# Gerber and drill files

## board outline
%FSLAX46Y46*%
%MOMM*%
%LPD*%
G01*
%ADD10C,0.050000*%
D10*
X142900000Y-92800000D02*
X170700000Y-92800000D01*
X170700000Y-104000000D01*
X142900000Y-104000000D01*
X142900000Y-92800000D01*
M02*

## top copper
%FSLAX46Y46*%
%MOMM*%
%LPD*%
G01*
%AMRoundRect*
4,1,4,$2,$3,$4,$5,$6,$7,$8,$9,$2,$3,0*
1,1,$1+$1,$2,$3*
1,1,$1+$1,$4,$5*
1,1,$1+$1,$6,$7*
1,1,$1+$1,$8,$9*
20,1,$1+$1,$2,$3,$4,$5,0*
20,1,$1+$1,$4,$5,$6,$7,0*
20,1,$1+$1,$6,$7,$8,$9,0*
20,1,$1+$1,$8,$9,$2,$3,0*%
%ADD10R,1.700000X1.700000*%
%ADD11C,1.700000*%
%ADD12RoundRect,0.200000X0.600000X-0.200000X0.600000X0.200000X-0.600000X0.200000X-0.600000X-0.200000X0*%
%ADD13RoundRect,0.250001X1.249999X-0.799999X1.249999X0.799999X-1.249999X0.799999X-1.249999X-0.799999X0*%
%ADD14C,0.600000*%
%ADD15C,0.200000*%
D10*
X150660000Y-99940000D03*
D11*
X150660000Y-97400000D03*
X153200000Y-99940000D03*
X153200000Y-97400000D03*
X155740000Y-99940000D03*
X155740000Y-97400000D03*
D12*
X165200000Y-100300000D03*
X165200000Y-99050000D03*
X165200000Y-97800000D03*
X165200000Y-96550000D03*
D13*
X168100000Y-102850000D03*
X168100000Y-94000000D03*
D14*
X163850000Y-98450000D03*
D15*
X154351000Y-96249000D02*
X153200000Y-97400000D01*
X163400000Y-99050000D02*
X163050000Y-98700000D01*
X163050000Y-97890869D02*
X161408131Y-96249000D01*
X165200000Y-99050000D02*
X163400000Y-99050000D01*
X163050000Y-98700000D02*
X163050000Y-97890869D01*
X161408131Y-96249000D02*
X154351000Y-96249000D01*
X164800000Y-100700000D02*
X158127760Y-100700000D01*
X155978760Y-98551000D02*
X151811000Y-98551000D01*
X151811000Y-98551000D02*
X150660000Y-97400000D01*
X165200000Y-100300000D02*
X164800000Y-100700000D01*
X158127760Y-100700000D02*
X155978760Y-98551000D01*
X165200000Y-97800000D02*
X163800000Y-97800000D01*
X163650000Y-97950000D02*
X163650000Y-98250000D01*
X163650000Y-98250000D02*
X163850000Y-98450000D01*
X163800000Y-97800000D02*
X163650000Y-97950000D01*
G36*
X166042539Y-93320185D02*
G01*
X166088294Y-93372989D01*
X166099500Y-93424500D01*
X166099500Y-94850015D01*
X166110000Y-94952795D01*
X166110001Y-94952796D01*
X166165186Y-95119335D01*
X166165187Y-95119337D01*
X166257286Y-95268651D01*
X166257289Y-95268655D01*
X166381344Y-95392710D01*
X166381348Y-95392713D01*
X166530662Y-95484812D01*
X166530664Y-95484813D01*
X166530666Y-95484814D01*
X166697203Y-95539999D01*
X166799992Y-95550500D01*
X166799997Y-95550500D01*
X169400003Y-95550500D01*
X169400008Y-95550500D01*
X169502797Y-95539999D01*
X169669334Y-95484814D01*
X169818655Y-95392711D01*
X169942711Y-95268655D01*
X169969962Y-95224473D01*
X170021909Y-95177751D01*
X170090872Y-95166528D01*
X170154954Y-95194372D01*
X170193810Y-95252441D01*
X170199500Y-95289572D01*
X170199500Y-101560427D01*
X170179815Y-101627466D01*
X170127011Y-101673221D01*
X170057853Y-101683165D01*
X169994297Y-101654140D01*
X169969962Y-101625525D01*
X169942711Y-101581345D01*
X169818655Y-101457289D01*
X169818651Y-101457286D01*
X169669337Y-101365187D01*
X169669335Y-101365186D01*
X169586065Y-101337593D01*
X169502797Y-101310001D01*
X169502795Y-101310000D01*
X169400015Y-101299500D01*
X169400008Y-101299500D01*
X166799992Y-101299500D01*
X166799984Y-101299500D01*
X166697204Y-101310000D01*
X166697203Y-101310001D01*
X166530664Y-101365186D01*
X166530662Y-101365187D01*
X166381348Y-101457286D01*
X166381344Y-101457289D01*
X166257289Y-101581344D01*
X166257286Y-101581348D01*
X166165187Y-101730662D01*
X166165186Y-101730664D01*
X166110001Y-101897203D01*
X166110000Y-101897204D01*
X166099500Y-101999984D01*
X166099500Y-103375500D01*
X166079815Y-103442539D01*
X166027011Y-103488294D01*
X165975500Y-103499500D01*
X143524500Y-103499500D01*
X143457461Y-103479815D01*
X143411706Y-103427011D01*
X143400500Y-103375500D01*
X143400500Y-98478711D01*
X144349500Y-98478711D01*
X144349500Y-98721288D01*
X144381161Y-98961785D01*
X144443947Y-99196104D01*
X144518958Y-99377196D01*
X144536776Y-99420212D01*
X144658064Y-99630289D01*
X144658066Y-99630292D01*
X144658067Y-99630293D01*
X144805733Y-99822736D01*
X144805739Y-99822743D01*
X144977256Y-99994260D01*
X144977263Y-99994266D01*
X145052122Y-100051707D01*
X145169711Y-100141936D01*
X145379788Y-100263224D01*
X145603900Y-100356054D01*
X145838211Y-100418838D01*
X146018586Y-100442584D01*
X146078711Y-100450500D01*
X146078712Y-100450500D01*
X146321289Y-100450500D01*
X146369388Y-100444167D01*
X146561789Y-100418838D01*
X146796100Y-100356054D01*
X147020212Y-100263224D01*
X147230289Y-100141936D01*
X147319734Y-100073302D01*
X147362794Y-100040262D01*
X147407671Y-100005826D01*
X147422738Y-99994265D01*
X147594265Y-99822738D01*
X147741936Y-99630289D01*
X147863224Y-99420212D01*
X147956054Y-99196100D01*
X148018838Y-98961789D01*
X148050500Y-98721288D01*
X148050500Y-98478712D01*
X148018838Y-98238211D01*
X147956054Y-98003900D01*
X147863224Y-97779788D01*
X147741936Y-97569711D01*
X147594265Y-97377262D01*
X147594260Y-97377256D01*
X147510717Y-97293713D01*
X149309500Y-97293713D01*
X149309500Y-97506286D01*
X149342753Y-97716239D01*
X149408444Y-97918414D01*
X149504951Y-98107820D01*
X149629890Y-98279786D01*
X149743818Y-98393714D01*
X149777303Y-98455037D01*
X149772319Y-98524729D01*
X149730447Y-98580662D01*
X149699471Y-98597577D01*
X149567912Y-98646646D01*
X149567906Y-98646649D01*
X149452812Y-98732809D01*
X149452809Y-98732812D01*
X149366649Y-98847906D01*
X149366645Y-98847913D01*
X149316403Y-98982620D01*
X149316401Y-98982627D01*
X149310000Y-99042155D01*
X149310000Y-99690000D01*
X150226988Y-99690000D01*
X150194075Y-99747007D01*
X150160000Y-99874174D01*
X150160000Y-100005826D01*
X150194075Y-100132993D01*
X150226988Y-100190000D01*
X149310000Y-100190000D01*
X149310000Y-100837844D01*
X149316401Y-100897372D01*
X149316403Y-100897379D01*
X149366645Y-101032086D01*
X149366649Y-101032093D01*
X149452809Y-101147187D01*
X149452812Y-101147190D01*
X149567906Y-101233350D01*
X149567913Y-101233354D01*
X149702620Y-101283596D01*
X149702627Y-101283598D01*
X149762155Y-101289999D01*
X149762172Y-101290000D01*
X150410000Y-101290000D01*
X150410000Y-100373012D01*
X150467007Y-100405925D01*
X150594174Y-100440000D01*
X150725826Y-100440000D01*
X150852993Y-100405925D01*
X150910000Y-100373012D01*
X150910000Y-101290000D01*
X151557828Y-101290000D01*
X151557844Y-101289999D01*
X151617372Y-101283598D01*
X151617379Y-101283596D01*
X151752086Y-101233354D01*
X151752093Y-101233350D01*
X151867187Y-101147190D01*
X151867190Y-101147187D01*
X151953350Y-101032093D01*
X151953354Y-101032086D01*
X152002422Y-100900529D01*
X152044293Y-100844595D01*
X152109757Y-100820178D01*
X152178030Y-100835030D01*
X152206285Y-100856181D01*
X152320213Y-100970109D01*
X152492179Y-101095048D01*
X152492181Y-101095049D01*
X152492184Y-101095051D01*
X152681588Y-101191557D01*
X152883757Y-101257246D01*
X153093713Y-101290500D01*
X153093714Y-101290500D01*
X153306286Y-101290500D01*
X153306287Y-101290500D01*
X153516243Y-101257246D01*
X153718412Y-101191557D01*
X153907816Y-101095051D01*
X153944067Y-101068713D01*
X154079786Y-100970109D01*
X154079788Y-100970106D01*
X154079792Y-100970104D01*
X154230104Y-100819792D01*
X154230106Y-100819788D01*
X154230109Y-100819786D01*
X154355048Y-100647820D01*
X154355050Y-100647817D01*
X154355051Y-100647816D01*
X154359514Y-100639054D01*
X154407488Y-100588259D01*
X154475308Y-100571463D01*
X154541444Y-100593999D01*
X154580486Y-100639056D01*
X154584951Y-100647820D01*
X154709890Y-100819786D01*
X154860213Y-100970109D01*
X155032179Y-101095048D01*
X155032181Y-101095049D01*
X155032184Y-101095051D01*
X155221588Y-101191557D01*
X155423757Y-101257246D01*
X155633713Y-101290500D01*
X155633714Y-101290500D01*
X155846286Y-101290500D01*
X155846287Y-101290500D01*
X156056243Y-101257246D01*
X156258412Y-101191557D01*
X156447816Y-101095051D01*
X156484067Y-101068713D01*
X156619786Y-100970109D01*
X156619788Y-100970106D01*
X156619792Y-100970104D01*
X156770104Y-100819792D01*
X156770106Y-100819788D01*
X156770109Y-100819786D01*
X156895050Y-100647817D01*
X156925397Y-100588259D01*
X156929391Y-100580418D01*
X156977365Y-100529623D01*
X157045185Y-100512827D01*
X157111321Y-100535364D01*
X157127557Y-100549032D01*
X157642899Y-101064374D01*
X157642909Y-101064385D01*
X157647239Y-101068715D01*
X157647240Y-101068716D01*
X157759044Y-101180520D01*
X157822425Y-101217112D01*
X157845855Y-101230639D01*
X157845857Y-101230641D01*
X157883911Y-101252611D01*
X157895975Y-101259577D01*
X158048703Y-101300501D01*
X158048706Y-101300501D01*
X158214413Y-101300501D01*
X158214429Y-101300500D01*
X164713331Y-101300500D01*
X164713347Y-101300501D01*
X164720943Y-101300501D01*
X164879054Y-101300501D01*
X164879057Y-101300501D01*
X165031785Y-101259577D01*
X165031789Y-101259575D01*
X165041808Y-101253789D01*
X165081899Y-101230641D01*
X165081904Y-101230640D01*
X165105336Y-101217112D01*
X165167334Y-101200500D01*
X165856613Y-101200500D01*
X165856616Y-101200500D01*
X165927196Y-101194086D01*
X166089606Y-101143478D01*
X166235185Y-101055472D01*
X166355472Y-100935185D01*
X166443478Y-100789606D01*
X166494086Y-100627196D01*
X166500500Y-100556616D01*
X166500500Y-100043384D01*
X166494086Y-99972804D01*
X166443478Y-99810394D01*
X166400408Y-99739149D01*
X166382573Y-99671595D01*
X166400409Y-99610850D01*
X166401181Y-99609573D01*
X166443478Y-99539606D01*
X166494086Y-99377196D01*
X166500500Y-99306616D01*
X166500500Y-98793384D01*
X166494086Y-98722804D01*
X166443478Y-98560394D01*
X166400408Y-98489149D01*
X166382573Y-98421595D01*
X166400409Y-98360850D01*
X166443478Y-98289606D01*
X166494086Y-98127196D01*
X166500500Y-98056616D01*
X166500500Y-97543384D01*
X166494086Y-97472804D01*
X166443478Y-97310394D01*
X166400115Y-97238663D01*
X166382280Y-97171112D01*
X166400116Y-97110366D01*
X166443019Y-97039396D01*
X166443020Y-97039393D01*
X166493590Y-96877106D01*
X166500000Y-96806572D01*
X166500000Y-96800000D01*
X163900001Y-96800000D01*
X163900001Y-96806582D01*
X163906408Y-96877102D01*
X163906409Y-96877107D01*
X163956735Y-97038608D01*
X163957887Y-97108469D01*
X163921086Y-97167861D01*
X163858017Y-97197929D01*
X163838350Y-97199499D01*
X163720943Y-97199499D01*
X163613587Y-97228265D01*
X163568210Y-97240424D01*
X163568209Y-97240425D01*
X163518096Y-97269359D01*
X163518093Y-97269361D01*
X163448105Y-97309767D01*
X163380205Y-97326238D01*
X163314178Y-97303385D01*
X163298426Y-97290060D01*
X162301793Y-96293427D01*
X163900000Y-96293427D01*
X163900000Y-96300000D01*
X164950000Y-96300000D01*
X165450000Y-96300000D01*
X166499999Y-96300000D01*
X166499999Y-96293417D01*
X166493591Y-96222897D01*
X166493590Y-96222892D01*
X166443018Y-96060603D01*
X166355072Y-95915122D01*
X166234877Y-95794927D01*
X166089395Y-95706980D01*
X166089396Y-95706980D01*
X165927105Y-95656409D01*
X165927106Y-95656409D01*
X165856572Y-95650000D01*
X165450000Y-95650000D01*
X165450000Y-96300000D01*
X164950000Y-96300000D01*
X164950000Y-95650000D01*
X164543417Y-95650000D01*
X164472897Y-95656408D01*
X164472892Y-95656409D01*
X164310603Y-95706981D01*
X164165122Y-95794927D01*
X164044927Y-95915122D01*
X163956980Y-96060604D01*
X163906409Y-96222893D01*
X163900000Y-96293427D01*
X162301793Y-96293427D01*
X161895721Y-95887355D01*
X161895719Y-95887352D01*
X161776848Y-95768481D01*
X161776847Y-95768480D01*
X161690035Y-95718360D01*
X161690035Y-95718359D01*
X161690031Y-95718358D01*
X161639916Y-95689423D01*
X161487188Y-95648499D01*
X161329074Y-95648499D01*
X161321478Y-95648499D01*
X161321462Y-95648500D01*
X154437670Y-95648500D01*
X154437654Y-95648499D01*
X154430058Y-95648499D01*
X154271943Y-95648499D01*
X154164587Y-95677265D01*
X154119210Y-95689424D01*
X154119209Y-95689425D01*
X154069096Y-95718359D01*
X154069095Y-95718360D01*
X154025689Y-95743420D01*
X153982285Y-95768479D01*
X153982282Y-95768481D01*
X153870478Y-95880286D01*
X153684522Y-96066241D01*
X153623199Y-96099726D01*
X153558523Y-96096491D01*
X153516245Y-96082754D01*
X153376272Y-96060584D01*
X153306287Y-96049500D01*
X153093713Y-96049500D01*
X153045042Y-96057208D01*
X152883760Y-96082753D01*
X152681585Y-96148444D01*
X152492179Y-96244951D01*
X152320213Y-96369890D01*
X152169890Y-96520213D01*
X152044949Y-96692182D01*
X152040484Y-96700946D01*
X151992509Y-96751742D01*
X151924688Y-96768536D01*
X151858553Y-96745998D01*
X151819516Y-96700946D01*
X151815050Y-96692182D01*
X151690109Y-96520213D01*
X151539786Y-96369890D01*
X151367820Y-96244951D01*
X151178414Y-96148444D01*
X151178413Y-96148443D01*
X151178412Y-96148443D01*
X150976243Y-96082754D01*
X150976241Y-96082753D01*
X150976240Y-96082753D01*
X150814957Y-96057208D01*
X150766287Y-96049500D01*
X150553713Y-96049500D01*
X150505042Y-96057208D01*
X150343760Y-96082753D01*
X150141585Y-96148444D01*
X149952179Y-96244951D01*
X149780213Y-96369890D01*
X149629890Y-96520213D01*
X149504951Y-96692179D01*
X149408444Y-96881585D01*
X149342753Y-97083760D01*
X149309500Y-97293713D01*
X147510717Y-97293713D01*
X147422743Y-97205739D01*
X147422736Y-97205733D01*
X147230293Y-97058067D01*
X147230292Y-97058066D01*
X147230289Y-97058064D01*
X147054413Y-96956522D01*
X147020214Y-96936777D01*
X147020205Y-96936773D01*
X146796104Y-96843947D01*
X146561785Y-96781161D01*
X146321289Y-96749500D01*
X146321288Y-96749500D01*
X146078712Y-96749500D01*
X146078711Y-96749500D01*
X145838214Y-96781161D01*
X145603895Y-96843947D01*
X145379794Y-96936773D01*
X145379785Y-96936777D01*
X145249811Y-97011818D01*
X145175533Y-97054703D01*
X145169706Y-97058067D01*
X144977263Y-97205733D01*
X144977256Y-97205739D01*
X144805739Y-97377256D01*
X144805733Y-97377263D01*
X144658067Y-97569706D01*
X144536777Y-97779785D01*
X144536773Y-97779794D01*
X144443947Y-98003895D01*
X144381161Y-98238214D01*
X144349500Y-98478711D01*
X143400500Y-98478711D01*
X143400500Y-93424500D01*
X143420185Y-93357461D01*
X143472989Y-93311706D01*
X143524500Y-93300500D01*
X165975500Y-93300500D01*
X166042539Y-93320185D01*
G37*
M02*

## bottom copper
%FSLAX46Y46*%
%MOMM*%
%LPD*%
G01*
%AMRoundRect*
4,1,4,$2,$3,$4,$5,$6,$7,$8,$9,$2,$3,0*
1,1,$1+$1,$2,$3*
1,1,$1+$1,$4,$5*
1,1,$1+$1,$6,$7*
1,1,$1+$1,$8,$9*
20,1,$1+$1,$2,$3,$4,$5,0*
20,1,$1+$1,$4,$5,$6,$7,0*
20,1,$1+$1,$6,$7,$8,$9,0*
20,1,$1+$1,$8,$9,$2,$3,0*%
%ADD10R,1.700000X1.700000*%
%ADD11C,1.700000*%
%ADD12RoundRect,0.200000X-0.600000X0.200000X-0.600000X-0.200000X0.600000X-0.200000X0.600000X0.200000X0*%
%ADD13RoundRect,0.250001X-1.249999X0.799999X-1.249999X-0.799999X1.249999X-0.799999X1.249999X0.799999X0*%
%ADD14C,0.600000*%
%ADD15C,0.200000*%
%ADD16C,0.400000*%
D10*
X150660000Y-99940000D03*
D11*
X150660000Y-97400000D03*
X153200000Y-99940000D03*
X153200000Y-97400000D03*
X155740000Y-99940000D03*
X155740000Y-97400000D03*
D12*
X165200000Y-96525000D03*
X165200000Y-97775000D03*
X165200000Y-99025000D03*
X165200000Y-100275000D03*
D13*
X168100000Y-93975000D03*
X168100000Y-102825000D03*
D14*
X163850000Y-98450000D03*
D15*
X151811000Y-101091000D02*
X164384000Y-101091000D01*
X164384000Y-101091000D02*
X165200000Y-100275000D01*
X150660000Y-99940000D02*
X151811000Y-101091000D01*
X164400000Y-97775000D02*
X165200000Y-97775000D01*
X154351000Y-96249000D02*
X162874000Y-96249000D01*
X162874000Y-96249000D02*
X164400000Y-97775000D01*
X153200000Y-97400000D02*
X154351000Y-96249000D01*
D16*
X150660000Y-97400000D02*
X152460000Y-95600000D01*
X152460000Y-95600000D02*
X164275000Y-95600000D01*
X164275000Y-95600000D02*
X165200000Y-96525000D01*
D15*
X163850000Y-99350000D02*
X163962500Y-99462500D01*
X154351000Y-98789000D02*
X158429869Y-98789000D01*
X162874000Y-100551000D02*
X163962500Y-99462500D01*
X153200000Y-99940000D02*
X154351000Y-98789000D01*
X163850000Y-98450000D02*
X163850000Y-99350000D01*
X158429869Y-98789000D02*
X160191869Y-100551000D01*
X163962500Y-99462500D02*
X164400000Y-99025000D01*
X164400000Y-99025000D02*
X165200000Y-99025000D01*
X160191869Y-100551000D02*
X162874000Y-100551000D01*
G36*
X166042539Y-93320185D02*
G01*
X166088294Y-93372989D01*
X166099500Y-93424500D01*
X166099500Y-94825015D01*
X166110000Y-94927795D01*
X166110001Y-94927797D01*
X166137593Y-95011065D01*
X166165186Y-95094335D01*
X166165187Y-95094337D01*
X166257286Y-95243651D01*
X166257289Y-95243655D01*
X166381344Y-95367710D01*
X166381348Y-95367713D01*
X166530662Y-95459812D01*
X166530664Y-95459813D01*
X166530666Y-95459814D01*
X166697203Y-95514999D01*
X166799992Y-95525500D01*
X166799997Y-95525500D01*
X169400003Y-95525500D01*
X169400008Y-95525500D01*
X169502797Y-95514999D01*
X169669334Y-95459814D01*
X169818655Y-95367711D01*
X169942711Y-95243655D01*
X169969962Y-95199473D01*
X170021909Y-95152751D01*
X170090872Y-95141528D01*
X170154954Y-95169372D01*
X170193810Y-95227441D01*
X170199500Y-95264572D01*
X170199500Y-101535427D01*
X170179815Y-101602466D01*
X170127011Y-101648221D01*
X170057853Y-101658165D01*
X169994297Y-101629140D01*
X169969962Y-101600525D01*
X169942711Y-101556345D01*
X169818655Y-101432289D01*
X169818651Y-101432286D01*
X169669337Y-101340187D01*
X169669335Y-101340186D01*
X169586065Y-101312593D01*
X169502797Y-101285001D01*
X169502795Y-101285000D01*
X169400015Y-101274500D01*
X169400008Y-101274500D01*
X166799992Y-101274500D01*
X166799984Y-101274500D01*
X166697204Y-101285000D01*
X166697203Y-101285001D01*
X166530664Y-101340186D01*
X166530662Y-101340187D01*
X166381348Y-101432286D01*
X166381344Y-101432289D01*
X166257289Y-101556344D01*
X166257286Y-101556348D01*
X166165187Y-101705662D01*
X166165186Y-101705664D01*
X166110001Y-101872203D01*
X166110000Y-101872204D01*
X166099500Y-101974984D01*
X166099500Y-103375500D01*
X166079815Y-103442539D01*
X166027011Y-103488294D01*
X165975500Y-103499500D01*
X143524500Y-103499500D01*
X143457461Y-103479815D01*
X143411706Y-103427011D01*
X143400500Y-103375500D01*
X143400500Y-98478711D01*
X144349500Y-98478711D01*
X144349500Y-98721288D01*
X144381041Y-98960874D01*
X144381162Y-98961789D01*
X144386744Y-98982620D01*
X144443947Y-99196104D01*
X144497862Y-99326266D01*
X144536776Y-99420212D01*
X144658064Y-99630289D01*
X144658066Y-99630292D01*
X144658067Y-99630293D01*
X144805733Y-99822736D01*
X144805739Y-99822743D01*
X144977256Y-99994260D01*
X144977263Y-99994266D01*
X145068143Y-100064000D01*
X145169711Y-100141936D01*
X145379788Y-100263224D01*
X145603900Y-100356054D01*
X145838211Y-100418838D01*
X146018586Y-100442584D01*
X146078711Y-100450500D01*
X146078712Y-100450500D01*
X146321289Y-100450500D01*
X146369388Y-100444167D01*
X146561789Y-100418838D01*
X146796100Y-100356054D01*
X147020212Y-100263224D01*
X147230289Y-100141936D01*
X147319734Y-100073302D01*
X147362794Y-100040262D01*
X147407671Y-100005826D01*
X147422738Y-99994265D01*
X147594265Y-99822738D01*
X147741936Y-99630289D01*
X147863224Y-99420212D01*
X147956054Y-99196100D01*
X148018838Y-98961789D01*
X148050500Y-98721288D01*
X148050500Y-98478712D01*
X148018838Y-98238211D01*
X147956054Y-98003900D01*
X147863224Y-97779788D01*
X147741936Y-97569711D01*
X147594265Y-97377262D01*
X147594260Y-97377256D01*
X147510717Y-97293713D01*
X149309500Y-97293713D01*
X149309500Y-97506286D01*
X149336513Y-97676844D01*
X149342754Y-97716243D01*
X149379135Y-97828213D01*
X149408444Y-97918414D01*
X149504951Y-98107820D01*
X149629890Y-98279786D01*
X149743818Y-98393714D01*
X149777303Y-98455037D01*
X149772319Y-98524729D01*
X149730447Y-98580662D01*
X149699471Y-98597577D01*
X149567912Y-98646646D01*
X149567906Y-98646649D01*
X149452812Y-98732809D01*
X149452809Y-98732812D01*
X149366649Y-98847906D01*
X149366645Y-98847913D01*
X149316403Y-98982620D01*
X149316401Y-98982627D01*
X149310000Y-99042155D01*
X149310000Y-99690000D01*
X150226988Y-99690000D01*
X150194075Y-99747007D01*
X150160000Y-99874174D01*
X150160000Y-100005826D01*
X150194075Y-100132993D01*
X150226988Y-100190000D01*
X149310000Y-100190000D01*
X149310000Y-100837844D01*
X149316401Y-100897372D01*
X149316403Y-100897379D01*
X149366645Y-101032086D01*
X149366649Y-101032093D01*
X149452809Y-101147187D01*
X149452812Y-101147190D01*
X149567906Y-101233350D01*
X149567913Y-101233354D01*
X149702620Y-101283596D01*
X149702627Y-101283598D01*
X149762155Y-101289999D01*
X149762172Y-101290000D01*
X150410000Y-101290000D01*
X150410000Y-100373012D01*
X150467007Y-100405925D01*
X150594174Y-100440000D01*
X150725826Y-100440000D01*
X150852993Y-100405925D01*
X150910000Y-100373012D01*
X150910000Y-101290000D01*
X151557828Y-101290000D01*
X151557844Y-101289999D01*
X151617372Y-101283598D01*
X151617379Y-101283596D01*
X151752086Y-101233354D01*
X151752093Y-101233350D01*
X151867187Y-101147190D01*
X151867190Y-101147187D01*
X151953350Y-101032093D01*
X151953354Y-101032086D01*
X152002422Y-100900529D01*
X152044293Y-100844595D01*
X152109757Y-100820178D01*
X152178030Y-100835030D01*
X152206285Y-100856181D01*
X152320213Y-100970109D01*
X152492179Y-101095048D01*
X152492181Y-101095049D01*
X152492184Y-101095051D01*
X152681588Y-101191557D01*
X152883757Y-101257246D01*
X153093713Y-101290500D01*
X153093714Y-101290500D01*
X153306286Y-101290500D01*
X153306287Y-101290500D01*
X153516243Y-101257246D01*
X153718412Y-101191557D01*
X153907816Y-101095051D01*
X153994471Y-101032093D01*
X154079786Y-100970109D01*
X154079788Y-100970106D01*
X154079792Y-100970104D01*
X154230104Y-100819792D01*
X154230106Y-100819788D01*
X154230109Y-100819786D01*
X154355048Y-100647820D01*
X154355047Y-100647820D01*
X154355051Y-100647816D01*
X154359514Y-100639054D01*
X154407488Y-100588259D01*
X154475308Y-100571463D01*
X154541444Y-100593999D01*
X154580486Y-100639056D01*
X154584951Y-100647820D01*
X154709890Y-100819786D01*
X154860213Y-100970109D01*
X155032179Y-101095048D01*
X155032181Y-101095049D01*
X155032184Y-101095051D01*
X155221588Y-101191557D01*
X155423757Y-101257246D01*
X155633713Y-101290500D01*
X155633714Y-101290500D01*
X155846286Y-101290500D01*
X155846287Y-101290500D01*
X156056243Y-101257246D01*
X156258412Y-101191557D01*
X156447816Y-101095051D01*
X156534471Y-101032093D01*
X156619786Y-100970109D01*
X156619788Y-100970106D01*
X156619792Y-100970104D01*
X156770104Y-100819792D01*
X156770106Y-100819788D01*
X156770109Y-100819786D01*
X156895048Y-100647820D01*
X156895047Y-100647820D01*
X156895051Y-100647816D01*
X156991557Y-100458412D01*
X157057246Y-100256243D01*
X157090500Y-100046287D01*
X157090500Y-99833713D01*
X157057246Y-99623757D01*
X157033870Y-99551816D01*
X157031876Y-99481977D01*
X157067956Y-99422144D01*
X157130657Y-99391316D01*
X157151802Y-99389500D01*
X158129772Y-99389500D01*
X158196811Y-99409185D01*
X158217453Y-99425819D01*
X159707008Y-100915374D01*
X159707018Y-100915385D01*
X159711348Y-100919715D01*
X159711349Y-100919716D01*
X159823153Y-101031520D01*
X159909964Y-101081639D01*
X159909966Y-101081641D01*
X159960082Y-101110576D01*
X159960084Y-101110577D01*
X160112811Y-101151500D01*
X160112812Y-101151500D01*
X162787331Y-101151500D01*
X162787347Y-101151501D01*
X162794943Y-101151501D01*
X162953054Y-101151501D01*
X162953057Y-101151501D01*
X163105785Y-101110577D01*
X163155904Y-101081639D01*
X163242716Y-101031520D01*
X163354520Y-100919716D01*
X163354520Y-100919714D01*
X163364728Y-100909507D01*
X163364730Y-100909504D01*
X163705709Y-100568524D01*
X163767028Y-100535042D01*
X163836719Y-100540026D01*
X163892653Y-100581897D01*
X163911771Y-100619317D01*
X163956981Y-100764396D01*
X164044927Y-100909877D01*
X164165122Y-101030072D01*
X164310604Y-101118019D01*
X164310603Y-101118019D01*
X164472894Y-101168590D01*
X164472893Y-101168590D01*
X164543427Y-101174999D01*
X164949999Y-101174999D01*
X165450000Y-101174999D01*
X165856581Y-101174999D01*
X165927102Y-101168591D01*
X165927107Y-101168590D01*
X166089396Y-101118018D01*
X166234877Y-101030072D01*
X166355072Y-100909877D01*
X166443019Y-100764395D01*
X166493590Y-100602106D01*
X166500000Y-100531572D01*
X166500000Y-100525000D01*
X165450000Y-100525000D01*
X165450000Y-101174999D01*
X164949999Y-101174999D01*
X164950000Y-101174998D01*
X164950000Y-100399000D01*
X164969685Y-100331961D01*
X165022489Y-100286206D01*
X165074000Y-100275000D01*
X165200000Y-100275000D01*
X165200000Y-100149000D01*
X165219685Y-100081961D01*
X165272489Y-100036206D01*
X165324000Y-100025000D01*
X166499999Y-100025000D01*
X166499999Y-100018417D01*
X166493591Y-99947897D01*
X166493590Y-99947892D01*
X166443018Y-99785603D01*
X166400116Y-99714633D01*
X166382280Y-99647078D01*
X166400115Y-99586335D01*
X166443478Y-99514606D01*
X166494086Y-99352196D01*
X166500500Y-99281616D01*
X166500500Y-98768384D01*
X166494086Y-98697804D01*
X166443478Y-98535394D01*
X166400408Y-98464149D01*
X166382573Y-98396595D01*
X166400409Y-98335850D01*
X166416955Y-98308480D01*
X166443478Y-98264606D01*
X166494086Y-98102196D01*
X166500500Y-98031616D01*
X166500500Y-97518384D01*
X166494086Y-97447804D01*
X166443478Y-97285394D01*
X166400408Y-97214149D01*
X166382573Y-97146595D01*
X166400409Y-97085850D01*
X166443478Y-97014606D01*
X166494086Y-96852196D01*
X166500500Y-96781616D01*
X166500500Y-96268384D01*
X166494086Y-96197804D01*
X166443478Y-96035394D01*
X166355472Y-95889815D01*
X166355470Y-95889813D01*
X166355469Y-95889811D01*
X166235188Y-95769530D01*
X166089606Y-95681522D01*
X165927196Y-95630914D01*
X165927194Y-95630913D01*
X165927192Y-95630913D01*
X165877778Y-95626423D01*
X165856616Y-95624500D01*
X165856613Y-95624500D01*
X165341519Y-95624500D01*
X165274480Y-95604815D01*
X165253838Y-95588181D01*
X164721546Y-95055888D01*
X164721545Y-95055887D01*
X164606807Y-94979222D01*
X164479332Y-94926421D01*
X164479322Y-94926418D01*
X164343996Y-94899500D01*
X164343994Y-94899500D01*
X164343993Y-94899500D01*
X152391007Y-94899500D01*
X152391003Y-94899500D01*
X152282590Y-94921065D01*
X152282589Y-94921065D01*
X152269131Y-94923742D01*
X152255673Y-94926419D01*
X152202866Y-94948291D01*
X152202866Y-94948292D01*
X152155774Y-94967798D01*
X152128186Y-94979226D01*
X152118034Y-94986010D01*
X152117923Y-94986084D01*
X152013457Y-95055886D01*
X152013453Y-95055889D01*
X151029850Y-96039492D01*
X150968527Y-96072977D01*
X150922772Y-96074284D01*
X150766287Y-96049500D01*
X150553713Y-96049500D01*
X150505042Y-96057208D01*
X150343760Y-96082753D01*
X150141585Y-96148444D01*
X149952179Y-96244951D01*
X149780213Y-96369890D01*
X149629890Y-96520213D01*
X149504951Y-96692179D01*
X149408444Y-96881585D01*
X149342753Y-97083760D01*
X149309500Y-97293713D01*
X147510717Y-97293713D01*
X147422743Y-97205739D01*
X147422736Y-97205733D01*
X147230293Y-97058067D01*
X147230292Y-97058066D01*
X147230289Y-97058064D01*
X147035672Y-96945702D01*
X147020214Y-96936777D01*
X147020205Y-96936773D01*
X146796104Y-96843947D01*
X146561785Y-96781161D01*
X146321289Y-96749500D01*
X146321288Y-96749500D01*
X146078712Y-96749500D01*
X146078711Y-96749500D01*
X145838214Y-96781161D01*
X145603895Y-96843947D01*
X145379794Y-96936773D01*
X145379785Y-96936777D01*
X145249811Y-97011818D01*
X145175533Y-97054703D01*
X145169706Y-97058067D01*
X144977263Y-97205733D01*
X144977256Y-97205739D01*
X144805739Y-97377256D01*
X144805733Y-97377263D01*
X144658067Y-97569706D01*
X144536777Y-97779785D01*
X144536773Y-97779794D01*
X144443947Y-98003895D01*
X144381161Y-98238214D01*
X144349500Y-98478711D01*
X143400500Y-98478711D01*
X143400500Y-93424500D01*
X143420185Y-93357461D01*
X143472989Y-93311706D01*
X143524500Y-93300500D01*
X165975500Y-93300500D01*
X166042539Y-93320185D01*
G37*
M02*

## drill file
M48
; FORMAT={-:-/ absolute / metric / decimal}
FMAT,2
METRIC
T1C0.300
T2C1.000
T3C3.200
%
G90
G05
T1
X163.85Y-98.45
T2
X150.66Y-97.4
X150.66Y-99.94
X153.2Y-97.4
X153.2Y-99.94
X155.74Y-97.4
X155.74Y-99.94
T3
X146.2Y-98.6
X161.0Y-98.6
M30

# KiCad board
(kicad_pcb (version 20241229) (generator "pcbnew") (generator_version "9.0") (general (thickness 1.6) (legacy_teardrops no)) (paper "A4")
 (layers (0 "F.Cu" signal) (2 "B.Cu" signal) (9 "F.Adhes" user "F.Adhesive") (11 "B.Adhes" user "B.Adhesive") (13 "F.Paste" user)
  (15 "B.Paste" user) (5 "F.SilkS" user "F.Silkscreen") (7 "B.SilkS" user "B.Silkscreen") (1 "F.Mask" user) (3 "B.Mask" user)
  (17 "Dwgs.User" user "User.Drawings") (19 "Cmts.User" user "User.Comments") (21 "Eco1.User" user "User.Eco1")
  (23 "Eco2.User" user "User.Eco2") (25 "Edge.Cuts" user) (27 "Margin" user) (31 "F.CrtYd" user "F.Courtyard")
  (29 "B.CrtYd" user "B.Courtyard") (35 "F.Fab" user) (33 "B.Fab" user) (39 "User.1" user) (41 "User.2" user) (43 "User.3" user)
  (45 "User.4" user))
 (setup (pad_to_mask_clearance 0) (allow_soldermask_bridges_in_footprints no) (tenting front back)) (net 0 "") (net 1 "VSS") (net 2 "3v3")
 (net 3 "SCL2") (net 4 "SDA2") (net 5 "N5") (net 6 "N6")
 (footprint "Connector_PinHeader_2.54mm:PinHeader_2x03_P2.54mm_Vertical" (layer "F.Cu") (at 150.66 99.94 90)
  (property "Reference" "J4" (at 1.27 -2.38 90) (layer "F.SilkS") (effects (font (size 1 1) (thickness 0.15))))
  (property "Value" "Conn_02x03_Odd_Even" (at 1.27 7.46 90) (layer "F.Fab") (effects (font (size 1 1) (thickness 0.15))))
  (pad "1" thru_hole rect (at 0 0 90) (size 1.7 1.7) (drill 1) (layers "*.Cu" "*.Mask") (remove_unused_layers no) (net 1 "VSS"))
  (pad "2" thru_hole circle (at 2.54 0 90) (size 1.7 1.7) (drill 1) (layers "*.Cu" "*.Mask") (remove_unused_layers no) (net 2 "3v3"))
  (pad "3" thru_hole circle (at 0 2.54 90) (size 1.7 1.7) (drill 1) (layers "*.Cu" "*.Mask") (remove_unused_layers no) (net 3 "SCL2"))
  (pad "4" thru_hole circle (at 2.54 2.54 90) (size 1.7 1.7) (drill 1) (layers "*.Cu" "*.Mask") (remove_unused_layers no) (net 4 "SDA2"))
  (pad "5" thru_hole circle (at 0 5.08 90) (size 1.7 1.7) (drill 1) (layers "*.Cu" "*.Mask") (remove_unused_layers no) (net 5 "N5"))
  (pad "6" thru_hole circle (at 2.54 5.08 90) (size 1.7 1.7) (drill 1) (layers "*.Cu" "*.Mask") (remove_unused_layers no) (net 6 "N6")))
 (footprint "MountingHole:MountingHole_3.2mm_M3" (layer "F.Cu") (at 161 98.6)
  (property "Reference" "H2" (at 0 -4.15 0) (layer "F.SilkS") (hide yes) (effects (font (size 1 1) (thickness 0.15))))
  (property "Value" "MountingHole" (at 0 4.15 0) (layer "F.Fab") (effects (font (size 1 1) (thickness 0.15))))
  (pad "" np_thru_hole circle (at 0 0) (size 3.2 3.2) (drill 3.2) (layers "*.Cu" "*.Mask")))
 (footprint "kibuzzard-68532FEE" (layer "F.Cu") (at 154.2 94.2)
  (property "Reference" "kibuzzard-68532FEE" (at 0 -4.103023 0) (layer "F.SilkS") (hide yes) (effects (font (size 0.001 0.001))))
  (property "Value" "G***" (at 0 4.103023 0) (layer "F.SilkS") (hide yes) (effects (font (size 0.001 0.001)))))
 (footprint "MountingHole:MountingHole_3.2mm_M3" (layer "F.Cu") (at 146.2 98.6)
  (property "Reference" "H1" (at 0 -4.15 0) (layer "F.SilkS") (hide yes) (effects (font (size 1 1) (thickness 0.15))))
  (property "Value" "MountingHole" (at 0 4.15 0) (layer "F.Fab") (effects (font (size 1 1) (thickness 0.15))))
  (pad "" np_thru_hole circle (at 0 0) (size 3.2 3.2) (drill 3.2) (layers "*.Cu" "*.Mask")))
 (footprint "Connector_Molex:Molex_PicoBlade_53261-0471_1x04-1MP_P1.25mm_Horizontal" (layer "F.Cu") (at 167.6 98.425 90)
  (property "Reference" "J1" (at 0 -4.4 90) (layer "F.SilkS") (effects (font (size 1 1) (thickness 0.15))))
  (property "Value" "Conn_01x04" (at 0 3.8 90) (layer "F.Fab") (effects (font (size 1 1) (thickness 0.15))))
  (pad "1" smd roundrect (at -1.875 -2.4 90) (size 0.8 1.6) (layers "F.Cu" "F.Mask" "F.Paste") (roundrect_rratio 0.25) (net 2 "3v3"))
  (pad "2" smd roundrect (at -0.625 -2.4 90) (size 0.8 1.6) (layers "F.Cu" "F.Mask" "F.Paste") (roundrect_rratio 0.25) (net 4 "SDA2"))
  (pad "3" smd roundrect (at 0.625 -2.4 90) (size 0.8 1.6) (layers "F.Cu" "F.Mask" "F.Paste") (roundrect_rratio 0.25) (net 3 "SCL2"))
  (pad "4" smd roundrect (at 1.875 -2.4 90) (size 0.8 1.6) (layers "F.Cu" "F.Mask" "F.Paste") (roundrect_rratio 0.25) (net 1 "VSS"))
  (pad "MP" smd roundrect (at -4.425 0.5 90) (size 2.1 3) (layers "F.Cu" "F.Mask" "F.Paste") (roundrect_rratio 0.119048))
  (pad "MP" smd roundrect (at 4.425 0.5 90) (size 2.1 3) (layers "F.Cu" "F.Mask" "F.Paste") (roundrect_rratio 0.119048)))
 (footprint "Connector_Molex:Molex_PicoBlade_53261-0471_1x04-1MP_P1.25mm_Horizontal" (layer "B.Cu") (at 167.6 98.4 -90)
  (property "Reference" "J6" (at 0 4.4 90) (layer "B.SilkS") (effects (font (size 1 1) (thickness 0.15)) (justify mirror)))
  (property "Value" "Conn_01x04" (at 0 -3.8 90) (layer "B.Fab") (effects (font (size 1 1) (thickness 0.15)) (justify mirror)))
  (pad "1" smd roundrect (at -1.875 2.4 270) (size 0.8 1.6) (layers "B.Cu" "B.Mask" "B.Paste") (roundrect_rratio 0.25) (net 2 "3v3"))
  (pad "2" smd roundrect (at -0.625 2.4 270) (size 0.8 1.6) (layers "B.Cu" "B.Mask" "B.Paste") (roundrect_rratio 0.25) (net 4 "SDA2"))
  (pad "3" smd roundrect (at 0.625 2.4 270) (size 0.8 1.6) (layers "B.Cu" "B.Mask" "B.Paste") (roundrect_rratio 0.25) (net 3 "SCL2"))
  (pad "4" smd roundrect (at 1.875 2.4 270) (size 0.8 1.6) (layers "B.Cu" "B.Mask" "B.Paste") (roundrect_rratio 0.25) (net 1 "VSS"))
  (pad "MP" smd roundrect (at -4.425 -0.5 270) (size 2.1 3) (layers "B.Cu" "B.Mask" "B.Paste") (roundrect_rratio 0.119048))
  (pad "MP" smd roundrect (at 4.425 -0.5 270) (size 2.1 3) (layers "B.Cu" "B.Mask" "B.Paste") (roundrect_rratio 0.119048)))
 (gr_rect (start 142.9 92.8) (end 170.7 104) (stroke (width 0.05) (type default)) (fill no) (layer "Edge.Cuts"))
 (segment (start 151.811 101.091) (end 164.384 101.091) (width 0.2) (layer "B.Cu") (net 1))
 (segment (start 164.384 101.091) (end 165.2 100.275) (width 0.2) (layer "B.Cu") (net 1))
 (segment (start 150.66 99.94) (end 151.811 101.091) (width 0.2) (layer "B.Cu") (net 1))
 (segment (start 154.351 96.249) (end 153.2 97.4) (width 0.2) (layer "F.Cu") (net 4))
 (segment (start 163.4 99.05) (end 163.05 98.7) (width 0.2) (layer "F.Cu") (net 4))
 (segment (start 163.05 97.890869) (end 161.408131 96.249) (width 0.2) (layer "F.Cu") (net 4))
 (segment (start 165.2 99.05) (end 163.4 99.05) (width 0.2) (layer "F.Cu") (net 4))
 (segment (start 163.05 98.7) (end 163.05 97.890869) (width 0.2) (layer "F.Cu") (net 4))
 (segment (start 161.408131 96.249) (end 154.351 96.249) (width 0.2) (layer "F.Cu") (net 4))
 (segment (start 164.4 97.775) (end 165.2 97.775) (width 0.2) (layer "B.Cu") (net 4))
 (segment (start 154.351 96.249) (end 162.874 96.249) (width 0.2) (layer "B.Cu") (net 4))
 (segment (start 162.874 96.249) (end 164.4 97.775) (width 0.2) (layer "B.Cu") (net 4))
 (segment (start 153.2 97.4) (end 154.351 96.249) (width 0.2) (layer "B.Cu") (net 4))
 (segment (start 164.8 100.7) (end 158.12776 100.7) (width 0.2) (layer "F.Cu") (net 2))
 (segment (start 155.97876 98.551) (end 151.811 98.551) (width 0.2) (layer "F.Cu") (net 2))
 (segment (start 151.811 98.551) (end 150.66 97.4) (width 0.2) (layer "F.Cu") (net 2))
 (segment (start 165.2 100.3) (end 164.8 100.7) (width 0.2) (layer "F.Cu") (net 2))
 (segment (start 158.12776 100.7) (end 155.97876 98.551) (width 0.2) (layer "F.Cu") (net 2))
 (segment (start 150.66 97.4) (end 152.46 95.6) (width 0.4) (layer "B.Cu") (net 2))
 (segment (start 152.46 95.6) (end 164.275 95.6) (width 0.4) (layer "B.Cu") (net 2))
 (segment (start 164.275 95.6) (end 165.2 96.525) (width 0.4) (layer "B.Cu") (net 2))
 (segment (start 165.2 97.8) (end 163.8 97.8) (width 0.2) (layer "F.Cu") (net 3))
 (segment (start 163.65 97.95) (end 163.65 98.25) (width 0.2) (layer "F.Cu") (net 3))
 (segment (start 163.65 98.25) (end 163.85 98.45) (width 0.2) (layer "F.Cu") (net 3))
 (segment (start 163.8 97.8) (end 163.65 97.95) (width 0.2) (layer "F.Cu") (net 3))
 (via (at 163.85 98.45) (size 0.6) (drill 0.3) (layers "F.Cu" "B.Cu") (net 3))
 (segment (start 163.85 99.35) (end 163.9625 99.4625) (width 0.2) (layer "B.Cu") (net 3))
 (segment (start 154.351 98.789) (end 158.429869 98.789) (width 0.2) (layer "B.Cu") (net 3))
 (segment (start 162.874 100.551) (end 163.9625 99.4625) (width 0.2) (layer "B.Cu") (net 3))
 (segment (start 153.2 99.94) (end 154.351 98.789) (width 0.2) (layer "B.Cu") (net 3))
 (segment (start 163.85 98.45) (end 163.85 99.35) (width 0.2) (layer "B.Cu") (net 3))
 (segment (start 158.429869 98.789) (end 160.191869 100.551) (width 0.2) (layer "B.Cu") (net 3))
 (segment (start 163.9625 99.4625) (end 164.4 99.025) (width 0.2) (layer "B.Cu") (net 3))
 (segment (start 164.4 99.025) (end 165.2 99.025) (width 0.2) (layer "B.Cu") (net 3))
 (segment (start 160.191869 100.551) (end 162.874 100.551) (width 0.2) (layer "B.Cu") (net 3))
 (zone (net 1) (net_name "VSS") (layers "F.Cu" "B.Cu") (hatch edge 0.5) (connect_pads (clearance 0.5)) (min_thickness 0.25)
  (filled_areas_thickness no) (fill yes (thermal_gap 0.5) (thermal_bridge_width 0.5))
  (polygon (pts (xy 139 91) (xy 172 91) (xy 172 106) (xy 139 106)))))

